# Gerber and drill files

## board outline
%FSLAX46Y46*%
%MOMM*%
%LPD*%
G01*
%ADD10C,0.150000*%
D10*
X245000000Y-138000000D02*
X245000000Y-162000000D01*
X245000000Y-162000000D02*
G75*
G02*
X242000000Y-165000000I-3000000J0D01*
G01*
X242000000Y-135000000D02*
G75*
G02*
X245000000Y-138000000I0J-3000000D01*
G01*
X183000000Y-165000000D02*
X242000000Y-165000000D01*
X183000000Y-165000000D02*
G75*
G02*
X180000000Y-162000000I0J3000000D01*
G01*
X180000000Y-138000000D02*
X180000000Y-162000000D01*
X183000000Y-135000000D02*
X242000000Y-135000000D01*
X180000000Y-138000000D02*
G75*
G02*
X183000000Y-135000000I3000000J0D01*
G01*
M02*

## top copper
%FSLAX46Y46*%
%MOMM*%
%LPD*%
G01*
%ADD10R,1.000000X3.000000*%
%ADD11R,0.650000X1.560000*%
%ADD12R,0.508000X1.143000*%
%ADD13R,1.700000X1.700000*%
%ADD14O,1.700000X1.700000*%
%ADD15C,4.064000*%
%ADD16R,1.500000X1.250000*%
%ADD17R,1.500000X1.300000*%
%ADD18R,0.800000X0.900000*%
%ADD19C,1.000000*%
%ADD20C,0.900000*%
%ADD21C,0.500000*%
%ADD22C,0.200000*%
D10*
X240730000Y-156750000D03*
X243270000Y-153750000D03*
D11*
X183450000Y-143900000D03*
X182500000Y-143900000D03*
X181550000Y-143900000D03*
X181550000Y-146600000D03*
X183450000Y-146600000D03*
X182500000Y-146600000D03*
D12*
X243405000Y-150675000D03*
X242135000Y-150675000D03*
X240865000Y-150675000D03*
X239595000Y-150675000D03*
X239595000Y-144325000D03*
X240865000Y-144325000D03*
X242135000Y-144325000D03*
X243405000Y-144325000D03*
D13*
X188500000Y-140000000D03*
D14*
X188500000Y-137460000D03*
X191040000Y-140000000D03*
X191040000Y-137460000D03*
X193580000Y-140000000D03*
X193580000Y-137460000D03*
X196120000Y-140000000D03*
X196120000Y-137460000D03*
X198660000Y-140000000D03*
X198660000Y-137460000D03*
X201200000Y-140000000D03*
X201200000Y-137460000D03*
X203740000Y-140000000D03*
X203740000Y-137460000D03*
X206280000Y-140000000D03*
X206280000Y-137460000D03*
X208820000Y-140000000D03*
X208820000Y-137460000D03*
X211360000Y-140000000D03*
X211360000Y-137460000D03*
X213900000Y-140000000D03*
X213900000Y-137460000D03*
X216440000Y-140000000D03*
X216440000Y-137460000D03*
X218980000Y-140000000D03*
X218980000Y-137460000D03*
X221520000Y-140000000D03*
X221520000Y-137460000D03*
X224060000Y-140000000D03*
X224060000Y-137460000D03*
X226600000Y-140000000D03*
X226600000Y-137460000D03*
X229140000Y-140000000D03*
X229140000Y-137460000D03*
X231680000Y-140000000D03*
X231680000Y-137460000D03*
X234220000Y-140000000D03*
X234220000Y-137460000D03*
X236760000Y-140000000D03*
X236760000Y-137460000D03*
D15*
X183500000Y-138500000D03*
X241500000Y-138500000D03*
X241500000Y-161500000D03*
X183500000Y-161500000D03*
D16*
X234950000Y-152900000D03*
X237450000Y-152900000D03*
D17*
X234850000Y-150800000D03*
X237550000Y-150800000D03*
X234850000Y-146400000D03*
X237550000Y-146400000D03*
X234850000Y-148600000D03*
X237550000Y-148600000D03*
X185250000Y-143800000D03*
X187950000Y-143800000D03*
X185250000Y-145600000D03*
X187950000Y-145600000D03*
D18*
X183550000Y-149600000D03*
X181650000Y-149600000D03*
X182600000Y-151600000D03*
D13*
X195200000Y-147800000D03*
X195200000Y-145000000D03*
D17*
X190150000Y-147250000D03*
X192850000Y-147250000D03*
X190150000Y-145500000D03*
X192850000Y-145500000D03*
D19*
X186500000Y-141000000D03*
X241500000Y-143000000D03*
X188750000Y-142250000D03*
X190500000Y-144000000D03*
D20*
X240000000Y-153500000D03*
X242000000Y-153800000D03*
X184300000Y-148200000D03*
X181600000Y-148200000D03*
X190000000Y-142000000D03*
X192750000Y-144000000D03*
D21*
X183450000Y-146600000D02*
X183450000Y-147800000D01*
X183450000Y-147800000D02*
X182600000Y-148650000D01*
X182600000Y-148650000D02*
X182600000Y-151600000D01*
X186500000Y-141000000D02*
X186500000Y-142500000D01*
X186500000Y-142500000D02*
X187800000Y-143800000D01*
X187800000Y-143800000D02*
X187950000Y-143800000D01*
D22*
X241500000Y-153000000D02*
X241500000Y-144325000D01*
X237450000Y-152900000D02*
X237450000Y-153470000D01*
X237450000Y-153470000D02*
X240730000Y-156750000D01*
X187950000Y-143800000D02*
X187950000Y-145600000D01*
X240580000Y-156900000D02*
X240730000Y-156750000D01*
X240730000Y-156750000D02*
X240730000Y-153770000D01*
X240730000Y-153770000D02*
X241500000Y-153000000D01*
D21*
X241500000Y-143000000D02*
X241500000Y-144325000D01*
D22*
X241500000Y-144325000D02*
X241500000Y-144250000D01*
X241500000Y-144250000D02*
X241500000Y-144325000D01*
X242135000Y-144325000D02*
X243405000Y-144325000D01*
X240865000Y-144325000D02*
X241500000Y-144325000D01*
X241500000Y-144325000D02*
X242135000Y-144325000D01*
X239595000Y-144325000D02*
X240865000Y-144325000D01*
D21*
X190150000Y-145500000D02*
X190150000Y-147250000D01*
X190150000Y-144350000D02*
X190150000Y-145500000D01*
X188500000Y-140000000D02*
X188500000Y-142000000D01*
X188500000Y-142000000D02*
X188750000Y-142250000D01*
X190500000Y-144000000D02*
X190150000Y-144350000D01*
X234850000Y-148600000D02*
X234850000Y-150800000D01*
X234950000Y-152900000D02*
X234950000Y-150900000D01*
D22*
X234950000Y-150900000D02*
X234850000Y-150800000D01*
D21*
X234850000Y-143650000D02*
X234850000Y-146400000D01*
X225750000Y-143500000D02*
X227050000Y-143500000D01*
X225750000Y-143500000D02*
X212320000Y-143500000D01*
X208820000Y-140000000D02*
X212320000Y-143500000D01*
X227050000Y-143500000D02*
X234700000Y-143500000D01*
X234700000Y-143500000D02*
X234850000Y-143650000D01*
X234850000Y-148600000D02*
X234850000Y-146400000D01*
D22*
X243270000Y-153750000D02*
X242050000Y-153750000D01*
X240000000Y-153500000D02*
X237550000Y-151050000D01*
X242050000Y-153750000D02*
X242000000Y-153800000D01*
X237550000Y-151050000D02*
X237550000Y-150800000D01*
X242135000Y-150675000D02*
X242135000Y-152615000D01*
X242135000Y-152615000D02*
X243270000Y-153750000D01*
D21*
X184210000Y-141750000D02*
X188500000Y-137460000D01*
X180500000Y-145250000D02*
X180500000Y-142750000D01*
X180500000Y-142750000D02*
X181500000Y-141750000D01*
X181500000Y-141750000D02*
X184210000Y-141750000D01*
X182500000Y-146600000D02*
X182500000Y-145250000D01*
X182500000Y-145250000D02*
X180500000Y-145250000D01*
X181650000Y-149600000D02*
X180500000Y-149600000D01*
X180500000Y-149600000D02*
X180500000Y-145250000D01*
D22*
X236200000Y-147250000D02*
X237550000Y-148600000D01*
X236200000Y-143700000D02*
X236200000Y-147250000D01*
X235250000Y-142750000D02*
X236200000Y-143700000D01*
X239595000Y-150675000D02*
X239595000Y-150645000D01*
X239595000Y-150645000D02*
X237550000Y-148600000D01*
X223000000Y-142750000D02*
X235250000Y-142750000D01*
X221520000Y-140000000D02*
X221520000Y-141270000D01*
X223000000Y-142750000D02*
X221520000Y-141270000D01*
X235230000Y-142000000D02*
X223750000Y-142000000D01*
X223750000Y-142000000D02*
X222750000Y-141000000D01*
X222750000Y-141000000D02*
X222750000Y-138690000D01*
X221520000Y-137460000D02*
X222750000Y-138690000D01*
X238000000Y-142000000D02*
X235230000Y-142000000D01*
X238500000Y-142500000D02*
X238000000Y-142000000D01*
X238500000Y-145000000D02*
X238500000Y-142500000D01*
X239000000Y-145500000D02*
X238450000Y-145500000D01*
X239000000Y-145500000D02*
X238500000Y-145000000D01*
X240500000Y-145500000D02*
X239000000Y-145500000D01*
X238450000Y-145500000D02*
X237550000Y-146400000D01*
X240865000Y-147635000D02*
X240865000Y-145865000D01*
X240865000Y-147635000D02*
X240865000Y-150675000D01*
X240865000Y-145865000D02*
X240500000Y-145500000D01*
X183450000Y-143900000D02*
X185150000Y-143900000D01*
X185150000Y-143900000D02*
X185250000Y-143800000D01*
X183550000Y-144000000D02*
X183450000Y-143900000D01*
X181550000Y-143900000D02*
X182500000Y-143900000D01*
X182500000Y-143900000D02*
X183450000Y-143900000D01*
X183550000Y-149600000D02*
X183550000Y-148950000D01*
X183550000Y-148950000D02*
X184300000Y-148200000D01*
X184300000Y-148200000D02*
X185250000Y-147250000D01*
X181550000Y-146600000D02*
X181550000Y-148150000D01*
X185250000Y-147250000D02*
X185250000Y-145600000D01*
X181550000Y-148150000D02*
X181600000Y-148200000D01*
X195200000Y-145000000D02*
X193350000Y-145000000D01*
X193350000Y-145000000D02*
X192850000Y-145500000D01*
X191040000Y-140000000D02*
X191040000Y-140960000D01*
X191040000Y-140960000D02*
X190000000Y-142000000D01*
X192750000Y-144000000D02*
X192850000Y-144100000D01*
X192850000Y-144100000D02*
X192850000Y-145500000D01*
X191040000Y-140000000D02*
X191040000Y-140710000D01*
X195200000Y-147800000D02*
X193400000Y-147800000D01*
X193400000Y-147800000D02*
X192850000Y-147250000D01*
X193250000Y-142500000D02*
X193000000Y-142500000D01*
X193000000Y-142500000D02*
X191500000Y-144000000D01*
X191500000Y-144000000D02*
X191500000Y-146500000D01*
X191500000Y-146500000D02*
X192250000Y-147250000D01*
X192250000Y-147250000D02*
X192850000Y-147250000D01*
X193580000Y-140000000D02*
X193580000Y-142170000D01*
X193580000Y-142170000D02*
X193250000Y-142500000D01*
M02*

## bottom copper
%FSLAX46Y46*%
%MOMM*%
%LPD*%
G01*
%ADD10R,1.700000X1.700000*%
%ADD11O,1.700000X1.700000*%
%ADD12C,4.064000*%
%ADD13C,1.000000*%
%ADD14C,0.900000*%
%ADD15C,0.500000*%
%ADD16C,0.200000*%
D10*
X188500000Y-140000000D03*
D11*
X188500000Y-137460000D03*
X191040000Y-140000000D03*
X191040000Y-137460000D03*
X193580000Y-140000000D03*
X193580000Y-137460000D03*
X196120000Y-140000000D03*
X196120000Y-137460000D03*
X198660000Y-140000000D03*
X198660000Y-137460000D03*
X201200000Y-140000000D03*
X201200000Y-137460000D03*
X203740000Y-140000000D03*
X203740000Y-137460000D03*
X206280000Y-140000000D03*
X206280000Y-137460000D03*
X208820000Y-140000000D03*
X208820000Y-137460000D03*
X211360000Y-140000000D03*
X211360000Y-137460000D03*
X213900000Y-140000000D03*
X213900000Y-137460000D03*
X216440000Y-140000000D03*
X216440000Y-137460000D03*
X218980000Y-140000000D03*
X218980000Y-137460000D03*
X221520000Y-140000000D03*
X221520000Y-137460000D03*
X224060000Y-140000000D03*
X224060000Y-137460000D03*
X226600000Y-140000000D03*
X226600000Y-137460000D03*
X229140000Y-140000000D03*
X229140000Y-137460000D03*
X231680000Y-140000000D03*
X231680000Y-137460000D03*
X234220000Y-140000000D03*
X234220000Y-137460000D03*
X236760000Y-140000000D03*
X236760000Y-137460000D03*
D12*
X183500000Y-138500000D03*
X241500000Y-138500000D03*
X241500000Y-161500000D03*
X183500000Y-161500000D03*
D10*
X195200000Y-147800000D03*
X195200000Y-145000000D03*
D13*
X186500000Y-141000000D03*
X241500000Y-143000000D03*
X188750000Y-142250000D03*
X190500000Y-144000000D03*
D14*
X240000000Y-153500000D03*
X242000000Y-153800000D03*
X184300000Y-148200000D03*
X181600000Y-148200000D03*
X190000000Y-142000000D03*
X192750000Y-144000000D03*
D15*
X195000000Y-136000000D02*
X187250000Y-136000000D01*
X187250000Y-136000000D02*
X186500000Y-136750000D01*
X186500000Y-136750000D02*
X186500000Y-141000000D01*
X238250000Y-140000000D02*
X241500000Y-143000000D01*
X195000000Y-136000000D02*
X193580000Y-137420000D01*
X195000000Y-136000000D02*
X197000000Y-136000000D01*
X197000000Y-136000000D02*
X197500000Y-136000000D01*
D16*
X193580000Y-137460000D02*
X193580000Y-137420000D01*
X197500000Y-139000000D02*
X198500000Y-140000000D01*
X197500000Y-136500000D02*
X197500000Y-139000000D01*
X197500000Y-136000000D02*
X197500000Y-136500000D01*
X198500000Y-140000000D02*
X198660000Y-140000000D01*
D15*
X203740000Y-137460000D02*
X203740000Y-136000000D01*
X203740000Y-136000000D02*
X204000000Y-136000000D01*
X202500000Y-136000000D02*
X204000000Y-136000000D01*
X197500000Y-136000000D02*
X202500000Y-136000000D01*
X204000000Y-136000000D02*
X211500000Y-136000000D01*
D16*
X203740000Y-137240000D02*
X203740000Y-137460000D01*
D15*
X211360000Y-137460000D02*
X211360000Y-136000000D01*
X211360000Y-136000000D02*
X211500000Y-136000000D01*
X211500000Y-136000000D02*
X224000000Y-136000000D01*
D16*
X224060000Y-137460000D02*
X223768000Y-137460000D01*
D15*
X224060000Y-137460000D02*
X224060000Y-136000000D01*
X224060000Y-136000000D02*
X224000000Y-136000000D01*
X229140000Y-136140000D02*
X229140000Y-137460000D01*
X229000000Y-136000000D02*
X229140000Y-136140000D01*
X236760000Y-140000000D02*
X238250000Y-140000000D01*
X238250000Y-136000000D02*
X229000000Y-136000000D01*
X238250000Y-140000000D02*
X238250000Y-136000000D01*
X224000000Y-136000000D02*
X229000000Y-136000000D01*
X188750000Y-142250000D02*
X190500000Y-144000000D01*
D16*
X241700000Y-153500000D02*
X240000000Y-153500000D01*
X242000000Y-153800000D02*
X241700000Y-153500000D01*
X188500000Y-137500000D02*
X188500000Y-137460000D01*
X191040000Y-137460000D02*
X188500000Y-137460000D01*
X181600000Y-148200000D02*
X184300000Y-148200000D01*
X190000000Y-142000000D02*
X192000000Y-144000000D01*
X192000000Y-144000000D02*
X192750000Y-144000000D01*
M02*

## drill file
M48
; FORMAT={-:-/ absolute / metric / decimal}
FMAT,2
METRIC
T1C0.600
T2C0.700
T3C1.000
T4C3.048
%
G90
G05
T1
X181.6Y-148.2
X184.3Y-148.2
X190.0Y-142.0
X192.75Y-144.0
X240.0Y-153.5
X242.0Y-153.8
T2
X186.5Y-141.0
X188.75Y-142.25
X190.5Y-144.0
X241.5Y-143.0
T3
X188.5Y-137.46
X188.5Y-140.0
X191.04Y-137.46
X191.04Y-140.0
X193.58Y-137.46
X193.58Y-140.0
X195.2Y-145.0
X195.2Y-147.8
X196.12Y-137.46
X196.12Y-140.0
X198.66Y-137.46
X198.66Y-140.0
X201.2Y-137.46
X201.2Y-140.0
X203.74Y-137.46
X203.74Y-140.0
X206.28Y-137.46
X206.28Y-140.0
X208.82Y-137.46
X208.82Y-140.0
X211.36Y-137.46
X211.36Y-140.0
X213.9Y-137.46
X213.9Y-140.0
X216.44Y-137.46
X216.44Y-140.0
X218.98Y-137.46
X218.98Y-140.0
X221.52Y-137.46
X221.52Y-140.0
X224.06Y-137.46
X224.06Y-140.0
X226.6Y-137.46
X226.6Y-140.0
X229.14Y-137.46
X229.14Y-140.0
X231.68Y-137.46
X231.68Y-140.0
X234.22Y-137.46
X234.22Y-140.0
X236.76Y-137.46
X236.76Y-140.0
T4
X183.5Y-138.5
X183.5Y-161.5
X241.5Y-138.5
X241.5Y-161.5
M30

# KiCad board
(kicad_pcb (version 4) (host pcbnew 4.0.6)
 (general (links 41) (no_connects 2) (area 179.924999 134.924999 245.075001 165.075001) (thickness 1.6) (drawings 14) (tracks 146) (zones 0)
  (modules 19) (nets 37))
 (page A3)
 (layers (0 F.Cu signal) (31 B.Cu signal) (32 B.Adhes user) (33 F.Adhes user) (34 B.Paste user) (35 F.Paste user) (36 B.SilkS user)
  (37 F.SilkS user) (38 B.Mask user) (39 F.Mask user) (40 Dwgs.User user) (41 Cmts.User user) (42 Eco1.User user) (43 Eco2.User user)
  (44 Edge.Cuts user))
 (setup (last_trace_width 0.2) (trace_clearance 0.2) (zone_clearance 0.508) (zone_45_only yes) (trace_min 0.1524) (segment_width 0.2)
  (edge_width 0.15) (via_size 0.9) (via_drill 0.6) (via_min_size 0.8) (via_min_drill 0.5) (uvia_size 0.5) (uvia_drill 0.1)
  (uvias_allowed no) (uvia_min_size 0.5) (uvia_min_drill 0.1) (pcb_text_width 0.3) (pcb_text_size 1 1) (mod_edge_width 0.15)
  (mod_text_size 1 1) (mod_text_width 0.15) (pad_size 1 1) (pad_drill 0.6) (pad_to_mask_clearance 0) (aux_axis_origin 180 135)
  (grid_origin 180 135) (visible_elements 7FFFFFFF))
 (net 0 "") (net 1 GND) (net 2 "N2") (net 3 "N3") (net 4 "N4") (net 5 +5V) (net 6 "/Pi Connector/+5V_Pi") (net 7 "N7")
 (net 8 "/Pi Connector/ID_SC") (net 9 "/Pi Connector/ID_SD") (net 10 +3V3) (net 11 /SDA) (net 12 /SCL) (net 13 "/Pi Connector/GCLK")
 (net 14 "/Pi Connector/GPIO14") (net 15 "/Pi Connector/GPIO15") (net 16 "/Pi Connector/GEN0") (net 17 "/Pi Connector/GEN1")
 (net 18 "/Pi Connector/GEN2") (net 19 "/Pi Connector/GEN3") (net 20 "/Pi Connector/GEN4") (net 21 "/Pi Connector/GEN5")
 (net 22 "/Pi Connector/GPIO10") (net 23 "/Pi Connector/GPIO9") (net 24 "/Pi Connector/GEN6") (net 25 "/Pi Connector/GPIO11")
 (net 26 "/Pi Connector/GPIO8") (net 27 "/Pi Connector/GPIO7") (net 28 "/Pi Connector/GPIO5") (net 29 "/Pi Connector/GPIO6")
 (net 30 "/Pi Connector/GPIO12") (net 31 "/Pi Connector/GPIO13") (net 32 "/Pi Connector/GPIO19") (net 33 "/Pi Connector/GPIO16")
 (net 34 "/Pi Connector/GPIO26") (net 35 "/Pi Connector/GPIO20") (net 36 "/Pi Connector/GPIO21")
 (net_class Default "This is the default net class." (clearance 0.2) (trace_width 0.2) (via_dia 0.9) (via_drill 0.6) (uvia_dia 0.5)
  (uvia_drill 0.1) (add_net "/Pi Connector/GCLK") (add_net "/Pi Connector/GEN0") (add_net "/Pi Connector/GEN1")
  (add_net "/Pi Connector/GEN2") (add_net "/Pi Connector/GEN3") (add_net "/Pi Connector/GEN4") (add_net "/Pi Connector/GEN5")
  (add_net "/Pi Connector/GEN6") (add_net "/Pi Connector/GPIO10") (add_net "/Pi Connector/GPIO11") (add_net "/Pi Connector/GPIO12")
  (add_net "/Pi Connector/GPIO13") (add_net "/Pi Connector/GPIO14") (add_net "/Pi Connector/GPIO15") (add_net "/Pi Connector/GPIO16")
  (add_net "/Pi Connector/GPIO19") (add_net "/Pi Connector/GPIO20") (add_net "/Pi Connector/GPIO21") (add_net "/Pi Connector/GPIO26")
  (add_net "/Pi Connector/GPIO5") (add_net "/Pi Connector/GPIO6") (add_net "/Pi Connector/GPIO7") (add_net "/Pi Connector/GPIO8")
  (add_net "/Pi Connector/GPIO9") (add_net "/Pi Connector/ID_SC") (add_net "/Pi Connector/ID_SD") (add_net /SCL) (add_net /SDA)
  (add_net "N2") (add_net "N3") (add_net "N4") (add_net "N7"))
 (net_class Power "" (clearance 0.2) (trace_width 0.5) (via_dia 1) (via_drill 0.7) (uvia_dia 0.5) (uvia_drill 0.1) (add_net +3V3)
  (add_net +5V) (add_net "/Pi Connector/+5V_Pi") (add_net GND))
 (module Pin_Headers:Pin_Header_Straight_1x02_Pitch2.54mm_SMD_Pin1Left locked (layer F.Cu) (at 242 155.25 90)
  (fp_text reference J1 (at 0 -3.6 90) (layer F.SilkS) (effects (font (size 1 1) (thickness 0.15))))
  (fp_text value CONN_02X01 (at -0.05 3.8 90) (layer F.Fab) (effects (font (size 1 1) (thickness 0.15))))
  (pad 1 smd rect (at -1.5 -1.27 90) (size 3 1) (layers F.Cu F.Paste F.Mask) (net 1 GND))
  (pad 2 smd rect (at 1.5 1.27 90) (size 3 1) (layers F.Cu F.Paste F.Mask) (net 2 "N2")))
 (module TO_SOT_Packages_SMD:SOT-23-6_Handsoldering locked (layer F.Cu) (at 182.5 145.25 270)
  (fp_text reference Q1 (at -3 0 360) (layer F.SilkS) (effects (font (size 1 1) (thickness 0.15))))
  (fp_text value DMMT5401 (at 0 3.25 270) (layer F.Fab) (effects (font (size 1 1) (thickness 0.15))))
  (pad 1 smd rect (at -1.35 -0.95 270) (size 1.56 0.65) (layers F.Cu F.Paste F.Mask) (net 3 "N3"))
  (pad 2 smd rect (at -1.35 0 270) (size 1.56 0.65) (layers F.Cu F.Paste F.Mask) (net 3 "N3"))
  (pad 3 smd rect (at -1.35 0.95 270) (size 1.56 0.65) (layers F.Cu F.Paste F.Mask) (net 3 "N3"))
  (pad 4 smd rect (at 1.35 0.95 270) (size 1.56 0.65) (layers F.Cu F.Paste F.Mask) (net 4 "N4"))
  (pad 6 smd rect (at 1.35 -0.95 270) (size 1.56 0.65) (layers F.Cu F.Paste F.Mask) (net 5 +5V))
  (pad 5 smd rect (at 1.35 0 270) (size 1.56 0.65) (layers F.Cu F.Paste F.Mask) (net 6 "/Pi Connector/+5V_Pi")))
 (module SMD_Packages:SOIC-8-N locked (layer F.Cu) (at 241.5 147.5 180)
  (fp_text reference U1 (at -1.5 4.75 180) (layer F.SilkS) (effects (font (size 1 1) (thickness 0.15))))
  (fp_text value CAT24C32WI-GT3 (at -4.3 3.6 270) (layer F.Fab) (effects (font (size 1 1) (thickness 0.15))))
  (pad 8 smd rect (at -1.905 -3.175 180) (size 0.508 1.143) (layers F.Cu F.Paste F.Mask) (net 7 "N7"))
  (pad 7 smd rect (at -0.635 -3.175 180) (size 0.508 1.143) (layers F.Cu F.Paste F.Mask) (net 2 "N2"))
  (pad 6 smd rect (at 0.635 -3.175 180) (size 0.508 1.143) (layers F.Cu F.Paste F.Mask) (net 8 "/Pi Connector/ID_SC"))
  (pad 5 smd rect (at 1.905 -3.175 180) (size 0.508 1.143) (layers F.Cu F.Paste F.Mask) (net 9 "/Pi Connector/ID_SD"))
  (pad 4 smd rect (at 1.905 3.175 180) (size 0.508 1.143) (layers F.Cu F.Paste F.Mask) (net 1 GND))
  (pad 3 smd rect (at 0.635 3.175 180) (size 0.508 1.143) (layers F.Cu F.Paste F.Mask) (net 1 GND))
  (pad 2 smd rect (at -0.635 3.175 180) (size 0.508 1.143) (layers F.Cu F.Paste F.Mask) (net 1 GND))
  (pad 1 smd rect (at -1.905 3.175 180) (size 0.508 1.143) (layers F.Cu F.Paste F.Mask) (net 1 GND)))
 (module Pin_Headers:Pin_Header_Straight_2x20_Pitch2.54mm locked (layer F.Cu) (at 188.5 140 90)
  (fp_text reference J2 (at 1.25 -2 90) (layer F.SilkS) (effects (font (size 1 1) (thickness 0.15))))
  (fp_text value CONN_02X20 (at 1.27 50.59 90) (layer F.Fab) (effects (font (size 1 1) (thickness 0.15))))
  (pad 1 thru_hole rect (at 0 0 90) (size 1.7 1.7) (drill 1) (layers *.Cu *.Mask) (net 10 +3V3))
  (pad 2 thru_hole oval (at 2.54 0 90) (size 1.7 1.7) (drill 1) (layers *.Cu *.Mask) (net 6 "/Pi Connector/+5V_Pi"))
  (pad 3 thru_hole oval (at 0 2.54 90) (size 1.7 1.7) (drill 1) (layers *.Cu *.Mask) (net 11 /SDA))
  (pad 4 thru_hole oval (at 2.54 2.54 90) (size 1.7 1.7) (drill 1) (layers *.Cu *.Mask) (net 6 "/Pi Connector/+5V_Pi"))
  (pad 5 thru_hole oval (at 0 5.08 90) (size 1.7 1.7) (drill 1) (layers *.Cu *.Mask) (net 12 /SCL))
  (pad 6 thru_hole oval (at 2.54 5.08 90) (size 1.7 1.7) (drill 1) (layers *.Cu *.Mask) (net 1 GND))
  (pad 7 thru_hole oval (at 0 7.62 90) (size 1.7 1.7) (drill 1) (layers *.Cu *.Mask) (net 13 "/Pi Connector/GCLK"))
  (pad 8 thru_hole oval (at 2.54 7.62 90) (size 1.7 1.7) (drill 1) (layers *.Cu *.Mask) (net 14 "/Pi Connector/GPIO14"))
  (pad 9 thru_hole oval (at 0 10.16 90) (size 1.7 1.7) (drill 1) (layers *.Cu *.Mask) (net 1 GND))
  (pad 10 thru_hole oval (at 2.54 10.16 90) (size 1.7 1.7) (drill 1) (layers *.Cu *.Mask) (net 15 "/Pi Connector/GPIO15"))
  (pad 11 thru_hole oval (at 0 12.7 90) (size 1.7 1.7) (drill 1) (layers *.Cu *.Mask) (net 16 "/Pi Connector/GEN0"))
  (pad 12 thru_hole oval (at 2.54 12.7 90) (size 1.7 1.7) (drill 1) (layers *.Cu *.Mask) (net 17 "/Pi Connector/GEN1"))
  (pad 13 thru_hole oval (at 0 15.24 90) (size 1.7 1.7) (drill 1) (layers *.Cu *.Mask) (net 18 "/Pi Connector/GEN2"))
  (pad 14 thru_hole oval (at 2.54 15.24 90) (size 1.7 1.7) (drill 1) (layers *.Cu *.Mask) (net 1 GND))
  (pad 15 thru_hole oval (at 0 17.78 90) (size 1.7 1.7) (drill 1) (layers *.Cu *.Mask) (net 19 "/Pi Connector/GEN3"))
  (pad 16 thru_hole oval (at 2.54 17.78 90) (size 1.7 1.7) (drill 1) (layers *.Cu *.Mask) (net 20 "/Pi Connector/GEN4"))
  (pad 17 thru_hole oval (at 0 20.32 90) (size 1.7 1.7) (drill 1) (layers *.Cu *.Mask) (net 10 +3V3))
  (pad 18 thru_hole oval (at 2.54 20.32 90) (size 1.7 1.7) (drill 1) (layers *.Cu *.Mask) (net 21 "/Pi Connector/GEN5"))
  (pad 19 thru_hole oval (at 0 22.86 90) (size 1.7 1.7) (drill 1) (layers *.Cu *.Mask) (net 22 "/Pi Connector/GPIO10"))
  (pad 20 thru_hole oval (at 2.54 22.86 90) (size 1.7 1.7) (drill 1) (layers *.Cu *.Mask) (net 1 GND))
  (pad 21 thru_hole oval (at 0 25.4 90) (size 1.7 1.7) (drill 1) (layers *.Cu *.Mask) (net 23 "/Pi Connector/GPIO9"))
  (pad 22 thru_hole oval (at 2.54 25.4 90) (size 1.7 1.7) (drill 1) (layers *.Cu *.Mask) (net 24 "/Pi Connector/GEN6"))
  (pad 23 thru_hole oval (at 0 27.94 90) (size 1.7 1.7) (drill 1) (layers *.Cu *.Mask) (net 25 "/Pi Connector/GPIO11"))
  (pad 24 thru_hole oval (at 2.54 27.94 90) (size 1.7 1.7) (drill 1) (layers *.Cu *.Mask) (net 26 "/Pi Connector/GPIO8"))
  (pad 25 thru_hole oval (at 0 30.48 90) (size 1.7 1.7) (drill 1) (layers *.Cu *.Mask) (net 1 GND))
  (pad 26 thru_hole oval (at 2.54 30.48 90) (size 1.7 1.7) (drill 1) (layers *.Cu *.Mask) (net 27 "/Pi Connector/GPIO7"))
  (pad 27 thru_hole oval (at 0 33.02 90) (size 1.7 1.7) (drill 1) (layers *.Cu *.Mask) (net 9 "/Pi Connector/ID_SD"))
  (pad 28 thru_hole oval (at 2.54 33.02 90) (size 1.7 1.7) (drill 1) (layers *.Cu *.Mask) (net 8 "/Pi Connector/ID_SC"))
  (pad 29 thru_hole oval (at 0 35.56 90) (size 1.7 1.7) (drill 1) (layers *.Cu *.Mask) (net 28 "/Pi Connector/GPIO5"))
  (pad 30 thru_hole oval (at 2.54 35.56 90) (size 1.7 1.7) (drill 1) (layers *.Cu *.Mask) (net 1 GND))
  (pad 31 thru_hole oval (at 0 38.1 90) (size 1.7 1.7) (drill 1) (layers *.Cu *.Mask) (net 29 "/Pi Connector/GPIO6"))
  (pad 32 thru_hole oval (at 2.54 38.1 90) (size 1.7 1.7) (drill 1) (layers *.Cu *.Mask) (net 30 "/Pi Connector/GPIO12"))
  (pad 33 thru_hole oval (at 0 40.64 90) (size 1.7 1.7) (drill 1) (layers *.Cu *.Mask) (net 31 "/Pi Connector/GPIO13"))
  (pad 34 thru_hole oval (at 2.54 40.64 90) (size 1.7 1.7) (drill 1) (layers *.Cu *.Mask) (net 1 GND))
  (pad 35 thru_hole oval (at 0 43.18 90) (size 1.7 1.7) (drill 1) (layers *.Cu *.Mask) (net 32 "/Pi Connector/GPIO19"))
  (pad 36 thru_hole oval (at 2.54 43.18 90) (size 1.7 1.7) (drill 1) (layers *.Cu *.Mask) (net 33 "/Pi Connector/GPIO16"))
  (pad 37 thru_hole oval (at 0 45.72 90) (size 1.7 1.7) (drill 1) (layers *.Cu *.Mask) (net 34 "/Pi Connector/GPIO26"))
  (pad 38 thru_hole oval (at 2.54 45.72 90) (size 1.7 1.7) (drill 1) (layers *.Cu *.Mask) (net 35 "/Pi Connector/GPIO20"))
  (pad 39 thru_hole oval (at 0 48.26 90) (size 1.7 1.7) (drill 1) (layers *.Cu *.Mask) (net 1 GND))
  (pad 40 thru_hole oval (at 2.54 48.26 90) (size 1.7 1.7) (drill 1) (layers *.Cu *.Mask) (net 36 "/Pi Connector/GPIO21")))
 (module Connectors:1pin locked (layer F.Cu) (at 183.5 138.5)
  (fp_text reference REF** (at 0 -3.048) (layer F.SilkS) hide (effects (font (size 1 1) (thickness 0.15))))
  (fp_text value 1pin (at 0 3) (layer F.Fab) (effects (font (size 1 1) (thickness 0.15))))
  (pad 1 thru_hole circle (at 0 0) (size 4.064 4.064) (drill 3.048) (layers *.Cu *.Mask)))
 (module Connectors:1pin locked (layer F.Cu) (at 241.5 138.5)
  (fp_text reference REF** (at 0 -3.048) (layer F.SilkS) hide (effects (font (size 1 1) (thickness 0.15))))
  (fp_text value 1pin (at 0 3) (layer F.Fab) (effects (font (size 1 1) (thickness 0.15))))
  (pad 1 thru_hole circle (at 0 0) (size 4.064 4.064) (drill 3.048) (layers *.Cu *.Mask)))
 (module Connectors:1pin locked (layer F.Cu) (at 241.5 161.5)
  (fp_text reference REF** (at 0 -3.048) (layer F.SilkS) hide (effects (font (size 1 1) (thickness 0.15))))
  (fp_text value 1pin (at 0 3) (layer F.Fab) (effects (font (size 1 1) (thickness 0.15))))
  (pad 1 thru_hole circle (at 0 0) (size 4.064 4.064) (drill 3.048) (layers *.Cu *.Mask)))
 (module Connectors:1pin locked (layer F.Cu) (at 183.5 161.5)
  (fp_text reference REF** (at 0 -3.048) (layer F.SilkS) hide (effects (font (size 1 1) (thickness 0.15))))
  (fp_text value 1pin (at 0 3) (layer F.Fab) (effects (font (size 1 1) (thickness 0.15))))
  (pad 1 thru_hole circle (at 0 0) (size 4.064 4.064) (drill 3.048) (layers *.Cu *.Mask)))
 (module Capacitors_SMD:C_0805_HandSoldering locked (layer F.Cu) (at 236.2 152.9)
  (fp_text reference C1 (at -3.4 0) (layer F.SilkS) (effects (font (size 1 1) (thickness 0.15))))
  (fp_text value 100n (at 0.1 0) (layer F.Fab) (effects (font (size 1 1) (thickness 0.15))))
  (pad 1 smd rect (at -1.25 0) (size 1.5 1.25) (layers F.Cu F.Paste F.Mask) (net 10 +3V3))
  (pad 2 smd rect (at 1.25 0) (size 1.5 1.25) (layers F.Cu F.Paste F.Mask) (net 1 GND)))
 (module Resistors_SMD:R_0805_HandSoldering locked (layer F.Cu) (at 236.2 150.8)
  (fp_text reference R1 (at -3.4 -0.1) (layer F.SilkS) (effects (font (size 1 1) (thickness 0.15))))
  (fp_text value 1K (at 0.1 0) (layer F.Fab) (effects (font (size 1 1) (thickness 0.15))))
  (pad 1 smd rect (at -1.35 0) (size 1.5 1.3) (layers F.Cu F.Paste F.Mask) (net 10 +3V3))
  (pad 2 smd rect (at 1.35 0) (size 1.5 1.3) (layers F.Cu F.Paste F.Mask) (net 2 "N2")))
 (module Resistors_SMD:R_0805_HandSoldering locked (layer F.Cu) (at 236.2 146.4)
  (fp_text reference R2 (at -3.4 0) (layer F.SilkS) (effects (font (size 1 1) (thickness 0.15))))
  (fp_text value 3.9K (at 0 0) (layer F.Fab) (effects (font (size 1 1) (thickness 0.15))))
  (pad 1 smd rect (at -1.35 0) (size 1.5 1.3) (layers F.Cu F.Paste F.Mask) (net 10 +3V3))
  (pad 2 smd rect (at 1.35 0) (size 1.5 1.3) (layers F.Cu F.Paste F.Mask) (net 8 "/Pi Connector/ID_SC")))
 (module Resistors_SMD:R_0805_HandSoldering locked (layer F.Cu) (at 236.2 148.6)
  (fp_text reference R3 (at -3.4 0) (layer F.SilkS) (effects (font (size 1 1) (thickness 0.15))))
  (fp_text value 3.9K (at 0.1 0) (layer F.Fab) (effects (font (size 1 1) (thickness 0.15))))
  (pad 1 smd rect (at -1.35 0) (size 1.5 1.3) (layers F.Cu F.Paste F.Mask) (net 10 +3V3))
  (pad 2 smd rect (at 1.35 0) (size 1.5 1.3) (layers F.Cu F.Paste F.Mask) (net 9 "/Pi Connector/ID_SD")))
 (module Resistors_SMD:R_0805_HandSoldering (layer F.Cu) (at 186.6 143.8)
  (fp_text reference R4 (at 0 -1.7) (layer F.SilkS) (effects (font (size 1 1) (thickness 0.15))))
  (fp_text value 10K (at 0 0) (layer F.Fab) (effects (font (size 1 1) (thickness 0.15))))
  (pad 1 smd rect (at -1.35 0) (size 1.5 1.3) (layers F.Cu F.Paste F.Mask) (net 3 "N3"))
  (pad 2 smd rect (at 1.35 0) (size 1.5 1.3) (layers F.Cu F.Paste F.Mask) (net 1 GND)))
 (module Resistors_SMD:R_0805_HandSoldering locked (layer F.Cu) (at 186.6 145.6)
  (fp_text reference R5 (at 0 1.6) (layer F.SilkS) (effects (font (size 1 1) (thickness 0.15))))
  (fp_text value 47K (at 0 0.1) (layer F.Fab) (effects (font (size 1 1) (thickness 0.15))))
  (pad 1 smd rect (at -1.35 0) (size 1.5 1.3) (layers F.Cu F.Paste F.Mask) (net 4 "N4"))
  (pad 2 smd rect (at 1.35 0) (size 1.5 1.3) (layers F.Cu F.Paste F.Mask) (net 1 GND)))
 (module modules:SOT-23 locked (layer F.Cu) (at 182.6 150.6 180)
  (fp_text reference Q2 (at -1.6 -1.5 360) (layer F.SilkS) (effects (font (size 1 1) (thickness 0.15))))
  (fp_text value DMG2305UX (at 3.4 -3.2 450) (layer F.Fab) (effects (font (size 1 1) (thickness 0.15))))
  (pad 1 smd rect (at -0.95 1 270) (size 0.9 0.8) (layers F.Cu F.Paste F.Mask) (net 4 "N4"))
  (pad 2 smd rect (at 0.95 1 270) (size 0.9 0.8) (layers F.Cu F.Paste F.Mask) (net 6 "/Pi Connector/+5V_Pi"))
  (pad 3 smd rect (at 0 -1 270) (size 0.9 0.8) (layers F.Cu F.Paste F.Mask) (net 5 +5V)))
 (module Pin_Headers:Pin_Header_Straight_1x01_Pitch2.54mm (layer F.Cu) (at 195.2 147.8)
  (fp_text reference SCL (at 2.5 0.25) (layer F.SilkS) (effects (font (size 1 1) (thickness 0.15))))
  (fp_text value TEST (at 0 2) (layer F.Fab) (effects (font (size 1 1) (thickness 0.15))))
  (pad 1 thru_hole rect (at 0 0) (size 1.7 1.7) (drill 1) (layers *.Cu *.Mask) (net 12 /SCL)))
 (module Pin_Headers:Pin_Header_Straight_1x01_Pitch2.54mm (layer F.Cu) (at 195.2 145)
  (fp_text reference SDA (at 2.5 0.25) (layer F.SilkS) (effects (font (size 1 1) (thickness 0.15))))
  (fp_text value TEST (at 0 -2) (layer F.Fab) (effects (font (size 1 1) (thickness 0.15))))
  (pad 1 thru_hole rect (at 0 0) (size 1.7 1.7) (drill 1) (layers *.Cu *.Mask) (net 11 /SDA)))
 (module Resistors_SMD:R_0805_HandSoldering (layer F.Cu) (at 191.5 147.25)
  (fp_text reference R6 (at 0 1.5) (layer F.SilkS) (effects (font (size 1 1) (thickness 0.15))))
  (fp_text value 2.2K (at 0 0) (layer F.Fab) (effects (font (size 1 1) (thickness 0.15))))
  (pad 1 smd rect (at -1.35 0) (size 1.5 1.3) (layers F.Cu F.Paste F.Mask) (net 10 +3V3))
  (pad 2 smd rect (at 1.35 0) (size 1.5 1.3) (layers F.Cu F.Paste F.Mask) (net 12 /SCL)))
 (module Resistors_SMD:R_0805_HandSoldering (layer F.Cu) (at 191.5 145.5)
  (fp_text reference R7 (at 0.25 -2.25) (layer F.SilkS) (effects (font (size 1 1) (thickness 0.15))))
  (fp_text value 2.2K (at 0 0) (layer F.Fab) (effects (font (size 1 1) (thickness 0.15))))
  (pad 1 smd rect (at -1.35 0) (size 1.5 1.3) (layers F.Cu F.Paste F.Mask) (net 10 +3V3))
  (pad 2 smd rect (at 1.35 0) (size 1.5 1.3) (layers F.Cu F.Paste F.Mask) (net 11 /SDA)))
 (gr_line (start 245 138) (end 245 162) (angle 90) (layer Edge.Cuts) (width 0.15))
 (gr_arc (start 242 162) (end 245 162) (angle 90) (layer Edge.Cuts) (width 0.15))
 (gr_arc (start 242 138) (end 242 135) (angle 90) (layer Edge.Cuts) (width 0.15))
 (gr_line (start 183 165) (end 242 165) (angle 90) (layer Edge.Cuts) (width 0.15))
 (gr_arc (start 183 162) (end 183 165) (angle 90) (layer Edge.Cuts) (width 0.15))
 (gr_line (start 180 138) (end 180 162) (angle 90) (layer Edge.Cuts) (width 0.15))
 (gr_line (start 183 135) (end 242 135) (angle 90) (layer Edge.Cuts) (width 0.15))
 (gr_arc (start 183 138) (end 180 138) (angle 90) (layer Edge.Cuts) (width 0.15))
 (segment (start 183.45 146.6) (end 183.45 147.8) (width 0.5) (layer F.Cu) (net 5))
 (segment (start 183.45 147.8) (end 182.6 148.65) (width 0.5) (layer F.Cu) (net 5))
 (segment (start 182.6 148.65) (end 182.6 151.6) (width 0.5) (layer F.Cu) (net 5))
 (segment (start 195 136) (end 187.25 136) (width 0.5) (layer B.Cu) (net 1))
 (segment (start 187.25 136) (end 186.5 136.75) (width 0.5) (layer B.Cu) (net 1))
 (segment (start 186.5 136.75) (end 186.5 141) (width 0.5) (layer B.Cu) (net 1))
 (via (at 186.5 141) (size 1) (drill 0.7) (layers F.Cu B.Cu) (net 1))
 (segment (start 186.5 141) (end 186.5 142.5) (width 0.5) (layer F.Cu) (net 1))
 (segment (start 186.5 142.5) (end 187.8 143.8) (width 0.5) (layer F.Cu) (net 1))
 (segment (start 187.8 143.8) (end 187.95 143.8) (width 0.5) (layer F.Cu) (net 1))
 (segment (start 241.5 153) (end 241.5 144.325) (width 0.2) (layer F.Cu) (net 1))
 (segment (start 237.45 152.9) (end 237.45 153.47) (width 0.2) (layer F.Cu) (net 1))
 (segment (start 237.45 153.47) (end 240.73 156.75) (width 0.2) (layer F.Cu) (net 1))
 (segment (start 187.95 143.8) (end 187.95 145.6) (width 0.2) (layer F.Cu) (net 1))
 (segment (start 240.58 156.9) (end 240.73 156.75) (width 0.2) (layer F.Cu) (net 1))
 (segment (start 240.73 156.75) (end 240.73 153.77) (width 0.2) (layer F.Cu) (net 1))
 (segment (start 240.73 153.77) (end 241.5 153) (width 0.2) (layer F.Cu) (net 1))
 (segment (start 241.5 143) (end 241.5 144.325) (width 0.5) (layer F.Cu) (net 1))
 (via (at 241.5 143) (size 1) (drill 0.7) (layers F.Cu B.Cu) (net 1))
 (segment (start 238.25 140) (end 241.5 143) (width 0.5) (layer B.Cu) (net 1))
 (segment (start 241.5 144.325) (end 241.5 144.25) (width 0.2) (layer F.Cu) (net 1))
 (segment (start 241.5 144.25) (end 241.5 144.325) (width 0.2) (layer F.Cu) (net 1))
 (segment (start 242.135 144.325) (end 243.405 144.325) (width 0.2) (layer F.Cu) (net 1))
 (segment (start 240.865 144.325) (end 241.5 144.325) (width 0.2) (layer F.Cu) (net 1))
 (segment (start 241.5 144.325) (end 242.135 144.325) (width 0.2) (layer F.Cu) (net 1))
 (segment (start 239.595 144.325) (end 240.865 144.325) (width 0.2) (layer F.Cu) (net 1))
 (segment (start 195 136) (end 193.58 137.42) (width 0.5) (layer B.Cu) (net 1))
 (segment (start 195 136) (end 197 136) (width 0.5) (layer B.Cu) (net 1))
 (segment (start 197 136) (end 197.5 136) (width 0.5) (layer B.Cu) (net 1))
 (segment (start 193.58 137.46) (end 193.58 137.42) (width 0.2) (layer B.Cu) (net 1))
 (segment (start 197.5 139) (end 198.5 140) (width 0.2) (layer B.Cu) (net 1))
 (segment (start 197.5 136.5) (end 197.5 139) (width 0.2) (layer B.Cu) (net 1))
 (segment (start 197.5 136) (end 197.5 136.5) (width 0.2) (layer B.Cu) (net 1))
 (segment (start 198.5 140) (end 198.66 140) (width 0.2) (layer B.Cu) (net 1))
 (segment (start 203.74 137.46) (end 203.74 136) (width 0.5) (layer B.Cu) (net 1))
 (segment (start 203.74 136) (end 204 136) (width 0.5) (layer B.Cu) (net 1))
 (segment (start 202.5 136) (end 204 136) (width 0.5) (layer B.Cu) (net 1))
 (segment (start 197.5 136) (end 202.5 136) (width 0.5) (layer B.Cu) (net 1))
 (segment (start 204 136) (end 211.5 136) (width 0.5) (layer B.Cu) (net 1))
 (segment (start 203.74 137.24) (end 203.74 137.46) (width 0.2) (layer B.Cu) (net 1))
 (segment (start 211.36 137.46) (end 211.36 136) (width 0.5) (layer B.Cu) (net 1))
 (segment (start 211.36 136) (end 211.5 136) (width 0.5) (layer B.Cu) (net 1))
 (segment (start 211.5 136) (end 224 136) (width 0.5) (layer B.Cu) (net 1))
 (segment (start 224.06 137.46) (end 223.768 137.46) (width 0.2) (layer B.Cu) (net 1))
 (segment (start 224.06 137.46) (end 224.06 136) (width 0.5) (layer B.Cu) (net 1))
 (segment (start 224.06 136) (end 224 136) (width 0.5) (layer B.Cu) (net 1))
 (segment (start 229.14 136.14) (end 229.14 137.46) (width 0.5) (layer B.Cu) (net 1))
 (segment (start 229 136) (end 229.14 136.14) (width 0.5) (layer B.Cu) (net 1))
 (segment (start 236.76 140) (end 238.25 140) (width 0.5) (layer B.Cu) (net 1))
 (segment (start 238.25 136) (end 229 136) (width 0.5) (layer B.Cu) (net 1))
 (segment (start 238.25 140) (end 238.25 136) (width 0.5) (layer B.Cu) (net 1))
 (segment (start 224 136) (end 229 136) (width 0.5) (layer B.Cu) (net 1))
 (segment (start 190.15 145.5) (end 190.15 147.25) (width 0.5) (layer F.Cu) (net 10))
 (segment (start 190.15 144.35) (end 190.15 145.5) (width 0.5) (layer F.Cu) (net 10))
 (segment (start 188.5 140) (end 188.5 142) (width 0.5) (layer F.Cu) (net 10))
 (segment (start 188.5 142) (end 188.75 142.25) (width 0.5) (layer F.Cu) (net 10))
 (via (at 188.75 142.25) (size 1) (drill 0.7) (layers F.Cu B.Cu) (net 10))
 (segment (start 188.75 142.25) (end 190.5 144) (width 0.5) (layer B.Cu) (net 10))
 (via (at 190.5 144) (size 1) (drill 0.7) (layers F.Cu B.Cu) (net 10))
 (segment (start 190.5 144) (end 190.15 144.35) (width 0.5) (layer F.Cu) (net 10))
 (segment (start 234.85 148.6) (end 234.85 150.8) (width 0.5) (layer F.Cu) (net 10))
 (segment (start 234.95 152.9) (end 234.95 150.9) (width 0.5) (layer F.Cu) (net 10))
 (segment (start 234.95 150.9) (end 234.85 150.8) (width 0.2) (layer F.Cu) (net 10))
 (segment (start 234.85 143.65) (end 234.85 146.4) (width 0.5) (layer F.Cu) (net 10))
 (segment (start 225.75 143.5) (end 227.05 143.5) (width 0.5) (layer F.Cu) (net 10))
 (segment (start 225.75 143.5) (end 212.32 143.5) (width 0.5) (layer F.Cu) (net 10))
 (segment (start 208.82 140) (end 212.32 143.5) (width 0.5) (layer F.Cu) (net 10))
 (segment (start 227.05 143.5) (end 234.7 143.5) (width 0.5) (layer F.Cu) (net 10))
 (segment (start 234.7 143.5) (end 234.85 143.65) (width 0.5) (layer F.Cu) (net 10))
 (segment (start 234.85 148.6) (end 234.85 146.4) (width 0.5) (layer F.Cu) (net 10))
 (segment (start 243.27 153.75) (end 242.05 153.75) (width 0.2) (layer F.Cu) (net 2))
 (segment (start 240 153.5) (end 237.55 151.05) (width 0.2) (layer F.Cu) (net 2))
 (via (at 240 153.5) (size 0.9) (drill 0.6) (layers F.Cu B.Cu) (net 2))
 (segment (start 241.7 153.5) (end 240 153.5) (width 0.2) (layer B.Cu) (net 2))
 (segment (start 242 153.8) (end 241.7 153.5) (width 0.2) (layer B.Cu) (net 2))
 (via (at 242 153.8) (size 0.9) (drill 0.6) (layers F.Cu B.Cu) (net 2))
 (segment (start 242.05 153.75) (end 242 153.8) (width 0.2) (layer F.Cu) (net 2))
 (segment (start 237.55 151.05) (end 237.55 150.8) (width 0.2) (layer F.Cu) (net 2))
 (segment (start 242.135 150.675) (end 242.135 152.615) (width 0.2) (layer F.Cu) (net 2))
 (segment (start 242.135 152.615) (end 243.27 153.75) (width 0.2) (layer F.Cu) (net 2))
 (segment (start 188.5 137.5) (end 188.5 137.46) (width 0.2) (layer B.Cu) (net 6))
 (segment (start 191.04 137.46) (end 188.5 137.46) (width 0.2) (layer B.Cu) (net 6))
 (segment (start 184.21 141.75) (end 188.5 137.46) (width 0.5) (layer F.Cu) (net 6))
 (segment (start 180.5 145.25) (end 180.5 142.75) (width 0.5) (layer F.Cu) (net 6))
 (segment (start 180.5 142.75) (end 181.5 141.75) (width 0.5) (layer F.Cu) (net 6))
 (segment (start 181.5 141.75) (end 184.21 141.75) (width 0.5) (layer F.Cu) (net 6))
 (segment (start 182.5 146.6) (end 182.5 145.25) (width 0.5) (layer F.Cu) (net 6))
 (segment (start 182.5 145.25) (end 180.5 145.25) (width 0.5) (layer F.Cu) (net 6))
 (segment (start 181.65 149.6) (end 180.5 149.6) (width 0.5) (layer F.Cu) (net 6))
 (segment (start 180.5 149.6) (end 180.5 145.25) (width 0.5) (layer F.Cu) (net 6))
 (segment (start 236.2 147.25) (end 237.55 148.6) (width 0.2) (layer F.Cu) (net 9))
 (segment (start 236.2 143.7) (end 236.2 147.25) (width 0.2) (layer F.Cu) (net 9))
 (segment (start 235.25 142.75) (end 236.2 143.7) (width 0.2) (layer F.Cu) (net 9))
 (segment (start 239.595 150.675) (end 239.595 150.645) (width 0.2) (layer F.Cu) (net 9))
 (segment (start 239.595 150.645) (end 237.55 148.6) (width 0.2) (layer F.Cu) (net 9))
 (segment (start 223 142.75) (end 235.25 142.75) (width 0.2) (layer F.Cu) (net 9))
 (segment (start 221.52 140) (end 221.52 141.27) (width 0.2) (layer F.Cu) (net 9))
 (segment (start 223 142.75) (end 221.52 141.27) (width 0.2) (layer F.Cu) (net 9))
 (segment (start 235.23 142) (end 223.75 142) (width 0.2) (layer F.Cu) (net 8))
 (segment (start 223.75 142) (end 222.75 141) (width 0.2) (layer F.Cu) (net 8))
 (segment (start 222.75 141) (end 222.75 138.69) (width 0.2) (layer F.Cu) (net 8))
 (segment (start 221.52 137.46) (end 222.75 138.69) (width 0.2) (layer F.Cu) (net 8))
 (segment (start 238 142) (end 235.23 142) (width 0.2) (layer F.Cu) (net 8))
 (segment (start 238.5 142.5) (end 238 142) (width 0.2) (layer F.Cu) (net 8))
 (segment (start 238.5 145) (end 238.5 142.5) (width 0.2) (layer F.Cu) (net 8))
 (segment (start 239 145.5) (end 238.45 145.5) (width 0.2) (layer F.Cu) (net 8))
 (segment (start 239 145.5) (end 238.5 145) (width 0.2) (layer F.Cu) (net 8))
 (segment (start 240.5 145.5) (end 239 145.5) (width 0.2) (layer F.Cu) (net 8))
 (segment (start 238.45 145.5) (end 237.55 146.4) (width 0.2) (layer F.Cu) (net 8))
 (segment (start 240.865 147.635) (end 240.865 145.865) (width 0.2) (layer F.Cu) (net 8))
 (segment (start 240.865 147.635) (end 240.865 150.675) (width 0.2) (layer F.Cu) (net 8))
 (segment (start 240.865 145.865) (end 240.5 145.5) (width 0.2) (layer F.Cu) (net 8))
 (segment (start 183.45 143.9) (end 185.15 143.9) (width 0.2) (layer F.Cu) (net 3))
 (segment (start 185.15 143.9) (end 185.25 143.8) (width 0.2) (layer F.Cu) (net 3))
 (segment (start 183.55 144) (end 183.45 143.9) (width 0.2) (layer F.Cu) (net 3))
 (segment (start 181.55 143.9) (end 182.5 143.9) (width 0.2) (layer F.Cu) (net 3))
 (segment (start 182.5 143.9) (end 183.45 143.9) (width 0.2) (layer F.Cu) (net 3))
 (segment (start 183.55 149.6) (end 183.55 148.95) (width 0.2) (layer F.Cu) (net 4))
 (segment (start 183.55 148.95) (end 184.3 148.2) (width 0.2) (layer F.Cu) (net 4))
 (segment (start 184.3 148.2) (end 185.25 147.25) (width 0.2) (layer F.Cu) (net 4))
 (via (at 184.3 148.2) (size 0.9) (drill 0.6) (layers F.Cu B.Cu) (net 4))
 (segment (start 181.6 148.2) (end 184.3 148.2) (width 0.2) (layer B.Cu) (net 4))
 (segment (start 181.55 146.6) (end 181.55 148.15) (width 0.2) (layer F.Cu) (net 4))
 (segment (start 185.25 147.25) (end 185.25 145.6) (width 0.2) (layer F.Cu) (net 4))
 (via (at 181.6 148.2) (size 0.9) (drill 0.6) (layers F.Cu B.Cu) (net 4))
 (segment (start 181.55 148.15) (end 181.6 148.2) (width 0.2) (layer F.Cu) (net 4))
 (segment (start 195.2 145) (end 193.35 145) (width 0.2) (layer F.Cu) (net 11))
 (segment (start 193.35 145) (end 192.85 145.5) (width 0.2) (layer F.Cu) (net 11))
 (segment (start 191.04 140) (end 191.04 140.96) (width 0.2) (layer F.Cu) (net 11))
 (segment (start 191.04 140.96) (end 190 142) (width 0.2) (layer F.Cu) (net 11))
 (via (at 190 142) (size 0.9) (drill 0.6) (layers F.Cu B.Cu) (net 11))
 (segment (start 190 142) (end 192 144) (width 0.2) (layer B.Cu) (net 11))
 (segment (start 192 144) (end 192.75 144) (width 0.2) (layer B.Cu) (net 11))
 (via (at 192.75 144) (size 0.9) (drill 0.6) (layers F.Cu B.Cu) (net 11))
 (segment (start 192.75 144) (end 192.85 144.1) (width 0.2) (layer F.Cu) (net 11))
 (segment (start 192.85 144.1) (end 192.85 145.5) (width 0.2) (layer F.Cu) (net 11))
 (segment (start 191.04 140) (end 191.04 140.71) (width 0.2) (layer F.Cu) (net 11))
 (segment (start 195.2 147.8) (end 193.4 147.8) (width 0.2) (layer F.Cu) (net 12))
 (segment (start 193.4 147.8) (end 192.85 147.25) (width 0.2) (layer F.Cu) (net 12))
 (segment (start 193.25 142.5) (end 193 142.5) (width 0.2) (layer F.Cu) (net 12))
 (segment (start 193 142.5) (end 191.5 144) (width 0.2) (layer F.Cu) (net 12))
 (segment (start 191.5 144) (end 191.5 146.5) (width 0.2) (layer F.Cu) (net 12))
 (segment (start 191.5 146.5) (end 192.25 147.25) (width 0.2) (layer F.Cu) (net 12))
 (segment (start 192.25 147.25) (end 192.85 147.25) (width 0.2) (layer F.Cu) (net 12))
 (segment (start 193.58 140) (end 193.58 142.17) (width 0.2) (layer F.Cu) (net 12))
 (segment (start 193.58 142.17) (end 193.25 142.5) (width 0.2) (layer F.Cu) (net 12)))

